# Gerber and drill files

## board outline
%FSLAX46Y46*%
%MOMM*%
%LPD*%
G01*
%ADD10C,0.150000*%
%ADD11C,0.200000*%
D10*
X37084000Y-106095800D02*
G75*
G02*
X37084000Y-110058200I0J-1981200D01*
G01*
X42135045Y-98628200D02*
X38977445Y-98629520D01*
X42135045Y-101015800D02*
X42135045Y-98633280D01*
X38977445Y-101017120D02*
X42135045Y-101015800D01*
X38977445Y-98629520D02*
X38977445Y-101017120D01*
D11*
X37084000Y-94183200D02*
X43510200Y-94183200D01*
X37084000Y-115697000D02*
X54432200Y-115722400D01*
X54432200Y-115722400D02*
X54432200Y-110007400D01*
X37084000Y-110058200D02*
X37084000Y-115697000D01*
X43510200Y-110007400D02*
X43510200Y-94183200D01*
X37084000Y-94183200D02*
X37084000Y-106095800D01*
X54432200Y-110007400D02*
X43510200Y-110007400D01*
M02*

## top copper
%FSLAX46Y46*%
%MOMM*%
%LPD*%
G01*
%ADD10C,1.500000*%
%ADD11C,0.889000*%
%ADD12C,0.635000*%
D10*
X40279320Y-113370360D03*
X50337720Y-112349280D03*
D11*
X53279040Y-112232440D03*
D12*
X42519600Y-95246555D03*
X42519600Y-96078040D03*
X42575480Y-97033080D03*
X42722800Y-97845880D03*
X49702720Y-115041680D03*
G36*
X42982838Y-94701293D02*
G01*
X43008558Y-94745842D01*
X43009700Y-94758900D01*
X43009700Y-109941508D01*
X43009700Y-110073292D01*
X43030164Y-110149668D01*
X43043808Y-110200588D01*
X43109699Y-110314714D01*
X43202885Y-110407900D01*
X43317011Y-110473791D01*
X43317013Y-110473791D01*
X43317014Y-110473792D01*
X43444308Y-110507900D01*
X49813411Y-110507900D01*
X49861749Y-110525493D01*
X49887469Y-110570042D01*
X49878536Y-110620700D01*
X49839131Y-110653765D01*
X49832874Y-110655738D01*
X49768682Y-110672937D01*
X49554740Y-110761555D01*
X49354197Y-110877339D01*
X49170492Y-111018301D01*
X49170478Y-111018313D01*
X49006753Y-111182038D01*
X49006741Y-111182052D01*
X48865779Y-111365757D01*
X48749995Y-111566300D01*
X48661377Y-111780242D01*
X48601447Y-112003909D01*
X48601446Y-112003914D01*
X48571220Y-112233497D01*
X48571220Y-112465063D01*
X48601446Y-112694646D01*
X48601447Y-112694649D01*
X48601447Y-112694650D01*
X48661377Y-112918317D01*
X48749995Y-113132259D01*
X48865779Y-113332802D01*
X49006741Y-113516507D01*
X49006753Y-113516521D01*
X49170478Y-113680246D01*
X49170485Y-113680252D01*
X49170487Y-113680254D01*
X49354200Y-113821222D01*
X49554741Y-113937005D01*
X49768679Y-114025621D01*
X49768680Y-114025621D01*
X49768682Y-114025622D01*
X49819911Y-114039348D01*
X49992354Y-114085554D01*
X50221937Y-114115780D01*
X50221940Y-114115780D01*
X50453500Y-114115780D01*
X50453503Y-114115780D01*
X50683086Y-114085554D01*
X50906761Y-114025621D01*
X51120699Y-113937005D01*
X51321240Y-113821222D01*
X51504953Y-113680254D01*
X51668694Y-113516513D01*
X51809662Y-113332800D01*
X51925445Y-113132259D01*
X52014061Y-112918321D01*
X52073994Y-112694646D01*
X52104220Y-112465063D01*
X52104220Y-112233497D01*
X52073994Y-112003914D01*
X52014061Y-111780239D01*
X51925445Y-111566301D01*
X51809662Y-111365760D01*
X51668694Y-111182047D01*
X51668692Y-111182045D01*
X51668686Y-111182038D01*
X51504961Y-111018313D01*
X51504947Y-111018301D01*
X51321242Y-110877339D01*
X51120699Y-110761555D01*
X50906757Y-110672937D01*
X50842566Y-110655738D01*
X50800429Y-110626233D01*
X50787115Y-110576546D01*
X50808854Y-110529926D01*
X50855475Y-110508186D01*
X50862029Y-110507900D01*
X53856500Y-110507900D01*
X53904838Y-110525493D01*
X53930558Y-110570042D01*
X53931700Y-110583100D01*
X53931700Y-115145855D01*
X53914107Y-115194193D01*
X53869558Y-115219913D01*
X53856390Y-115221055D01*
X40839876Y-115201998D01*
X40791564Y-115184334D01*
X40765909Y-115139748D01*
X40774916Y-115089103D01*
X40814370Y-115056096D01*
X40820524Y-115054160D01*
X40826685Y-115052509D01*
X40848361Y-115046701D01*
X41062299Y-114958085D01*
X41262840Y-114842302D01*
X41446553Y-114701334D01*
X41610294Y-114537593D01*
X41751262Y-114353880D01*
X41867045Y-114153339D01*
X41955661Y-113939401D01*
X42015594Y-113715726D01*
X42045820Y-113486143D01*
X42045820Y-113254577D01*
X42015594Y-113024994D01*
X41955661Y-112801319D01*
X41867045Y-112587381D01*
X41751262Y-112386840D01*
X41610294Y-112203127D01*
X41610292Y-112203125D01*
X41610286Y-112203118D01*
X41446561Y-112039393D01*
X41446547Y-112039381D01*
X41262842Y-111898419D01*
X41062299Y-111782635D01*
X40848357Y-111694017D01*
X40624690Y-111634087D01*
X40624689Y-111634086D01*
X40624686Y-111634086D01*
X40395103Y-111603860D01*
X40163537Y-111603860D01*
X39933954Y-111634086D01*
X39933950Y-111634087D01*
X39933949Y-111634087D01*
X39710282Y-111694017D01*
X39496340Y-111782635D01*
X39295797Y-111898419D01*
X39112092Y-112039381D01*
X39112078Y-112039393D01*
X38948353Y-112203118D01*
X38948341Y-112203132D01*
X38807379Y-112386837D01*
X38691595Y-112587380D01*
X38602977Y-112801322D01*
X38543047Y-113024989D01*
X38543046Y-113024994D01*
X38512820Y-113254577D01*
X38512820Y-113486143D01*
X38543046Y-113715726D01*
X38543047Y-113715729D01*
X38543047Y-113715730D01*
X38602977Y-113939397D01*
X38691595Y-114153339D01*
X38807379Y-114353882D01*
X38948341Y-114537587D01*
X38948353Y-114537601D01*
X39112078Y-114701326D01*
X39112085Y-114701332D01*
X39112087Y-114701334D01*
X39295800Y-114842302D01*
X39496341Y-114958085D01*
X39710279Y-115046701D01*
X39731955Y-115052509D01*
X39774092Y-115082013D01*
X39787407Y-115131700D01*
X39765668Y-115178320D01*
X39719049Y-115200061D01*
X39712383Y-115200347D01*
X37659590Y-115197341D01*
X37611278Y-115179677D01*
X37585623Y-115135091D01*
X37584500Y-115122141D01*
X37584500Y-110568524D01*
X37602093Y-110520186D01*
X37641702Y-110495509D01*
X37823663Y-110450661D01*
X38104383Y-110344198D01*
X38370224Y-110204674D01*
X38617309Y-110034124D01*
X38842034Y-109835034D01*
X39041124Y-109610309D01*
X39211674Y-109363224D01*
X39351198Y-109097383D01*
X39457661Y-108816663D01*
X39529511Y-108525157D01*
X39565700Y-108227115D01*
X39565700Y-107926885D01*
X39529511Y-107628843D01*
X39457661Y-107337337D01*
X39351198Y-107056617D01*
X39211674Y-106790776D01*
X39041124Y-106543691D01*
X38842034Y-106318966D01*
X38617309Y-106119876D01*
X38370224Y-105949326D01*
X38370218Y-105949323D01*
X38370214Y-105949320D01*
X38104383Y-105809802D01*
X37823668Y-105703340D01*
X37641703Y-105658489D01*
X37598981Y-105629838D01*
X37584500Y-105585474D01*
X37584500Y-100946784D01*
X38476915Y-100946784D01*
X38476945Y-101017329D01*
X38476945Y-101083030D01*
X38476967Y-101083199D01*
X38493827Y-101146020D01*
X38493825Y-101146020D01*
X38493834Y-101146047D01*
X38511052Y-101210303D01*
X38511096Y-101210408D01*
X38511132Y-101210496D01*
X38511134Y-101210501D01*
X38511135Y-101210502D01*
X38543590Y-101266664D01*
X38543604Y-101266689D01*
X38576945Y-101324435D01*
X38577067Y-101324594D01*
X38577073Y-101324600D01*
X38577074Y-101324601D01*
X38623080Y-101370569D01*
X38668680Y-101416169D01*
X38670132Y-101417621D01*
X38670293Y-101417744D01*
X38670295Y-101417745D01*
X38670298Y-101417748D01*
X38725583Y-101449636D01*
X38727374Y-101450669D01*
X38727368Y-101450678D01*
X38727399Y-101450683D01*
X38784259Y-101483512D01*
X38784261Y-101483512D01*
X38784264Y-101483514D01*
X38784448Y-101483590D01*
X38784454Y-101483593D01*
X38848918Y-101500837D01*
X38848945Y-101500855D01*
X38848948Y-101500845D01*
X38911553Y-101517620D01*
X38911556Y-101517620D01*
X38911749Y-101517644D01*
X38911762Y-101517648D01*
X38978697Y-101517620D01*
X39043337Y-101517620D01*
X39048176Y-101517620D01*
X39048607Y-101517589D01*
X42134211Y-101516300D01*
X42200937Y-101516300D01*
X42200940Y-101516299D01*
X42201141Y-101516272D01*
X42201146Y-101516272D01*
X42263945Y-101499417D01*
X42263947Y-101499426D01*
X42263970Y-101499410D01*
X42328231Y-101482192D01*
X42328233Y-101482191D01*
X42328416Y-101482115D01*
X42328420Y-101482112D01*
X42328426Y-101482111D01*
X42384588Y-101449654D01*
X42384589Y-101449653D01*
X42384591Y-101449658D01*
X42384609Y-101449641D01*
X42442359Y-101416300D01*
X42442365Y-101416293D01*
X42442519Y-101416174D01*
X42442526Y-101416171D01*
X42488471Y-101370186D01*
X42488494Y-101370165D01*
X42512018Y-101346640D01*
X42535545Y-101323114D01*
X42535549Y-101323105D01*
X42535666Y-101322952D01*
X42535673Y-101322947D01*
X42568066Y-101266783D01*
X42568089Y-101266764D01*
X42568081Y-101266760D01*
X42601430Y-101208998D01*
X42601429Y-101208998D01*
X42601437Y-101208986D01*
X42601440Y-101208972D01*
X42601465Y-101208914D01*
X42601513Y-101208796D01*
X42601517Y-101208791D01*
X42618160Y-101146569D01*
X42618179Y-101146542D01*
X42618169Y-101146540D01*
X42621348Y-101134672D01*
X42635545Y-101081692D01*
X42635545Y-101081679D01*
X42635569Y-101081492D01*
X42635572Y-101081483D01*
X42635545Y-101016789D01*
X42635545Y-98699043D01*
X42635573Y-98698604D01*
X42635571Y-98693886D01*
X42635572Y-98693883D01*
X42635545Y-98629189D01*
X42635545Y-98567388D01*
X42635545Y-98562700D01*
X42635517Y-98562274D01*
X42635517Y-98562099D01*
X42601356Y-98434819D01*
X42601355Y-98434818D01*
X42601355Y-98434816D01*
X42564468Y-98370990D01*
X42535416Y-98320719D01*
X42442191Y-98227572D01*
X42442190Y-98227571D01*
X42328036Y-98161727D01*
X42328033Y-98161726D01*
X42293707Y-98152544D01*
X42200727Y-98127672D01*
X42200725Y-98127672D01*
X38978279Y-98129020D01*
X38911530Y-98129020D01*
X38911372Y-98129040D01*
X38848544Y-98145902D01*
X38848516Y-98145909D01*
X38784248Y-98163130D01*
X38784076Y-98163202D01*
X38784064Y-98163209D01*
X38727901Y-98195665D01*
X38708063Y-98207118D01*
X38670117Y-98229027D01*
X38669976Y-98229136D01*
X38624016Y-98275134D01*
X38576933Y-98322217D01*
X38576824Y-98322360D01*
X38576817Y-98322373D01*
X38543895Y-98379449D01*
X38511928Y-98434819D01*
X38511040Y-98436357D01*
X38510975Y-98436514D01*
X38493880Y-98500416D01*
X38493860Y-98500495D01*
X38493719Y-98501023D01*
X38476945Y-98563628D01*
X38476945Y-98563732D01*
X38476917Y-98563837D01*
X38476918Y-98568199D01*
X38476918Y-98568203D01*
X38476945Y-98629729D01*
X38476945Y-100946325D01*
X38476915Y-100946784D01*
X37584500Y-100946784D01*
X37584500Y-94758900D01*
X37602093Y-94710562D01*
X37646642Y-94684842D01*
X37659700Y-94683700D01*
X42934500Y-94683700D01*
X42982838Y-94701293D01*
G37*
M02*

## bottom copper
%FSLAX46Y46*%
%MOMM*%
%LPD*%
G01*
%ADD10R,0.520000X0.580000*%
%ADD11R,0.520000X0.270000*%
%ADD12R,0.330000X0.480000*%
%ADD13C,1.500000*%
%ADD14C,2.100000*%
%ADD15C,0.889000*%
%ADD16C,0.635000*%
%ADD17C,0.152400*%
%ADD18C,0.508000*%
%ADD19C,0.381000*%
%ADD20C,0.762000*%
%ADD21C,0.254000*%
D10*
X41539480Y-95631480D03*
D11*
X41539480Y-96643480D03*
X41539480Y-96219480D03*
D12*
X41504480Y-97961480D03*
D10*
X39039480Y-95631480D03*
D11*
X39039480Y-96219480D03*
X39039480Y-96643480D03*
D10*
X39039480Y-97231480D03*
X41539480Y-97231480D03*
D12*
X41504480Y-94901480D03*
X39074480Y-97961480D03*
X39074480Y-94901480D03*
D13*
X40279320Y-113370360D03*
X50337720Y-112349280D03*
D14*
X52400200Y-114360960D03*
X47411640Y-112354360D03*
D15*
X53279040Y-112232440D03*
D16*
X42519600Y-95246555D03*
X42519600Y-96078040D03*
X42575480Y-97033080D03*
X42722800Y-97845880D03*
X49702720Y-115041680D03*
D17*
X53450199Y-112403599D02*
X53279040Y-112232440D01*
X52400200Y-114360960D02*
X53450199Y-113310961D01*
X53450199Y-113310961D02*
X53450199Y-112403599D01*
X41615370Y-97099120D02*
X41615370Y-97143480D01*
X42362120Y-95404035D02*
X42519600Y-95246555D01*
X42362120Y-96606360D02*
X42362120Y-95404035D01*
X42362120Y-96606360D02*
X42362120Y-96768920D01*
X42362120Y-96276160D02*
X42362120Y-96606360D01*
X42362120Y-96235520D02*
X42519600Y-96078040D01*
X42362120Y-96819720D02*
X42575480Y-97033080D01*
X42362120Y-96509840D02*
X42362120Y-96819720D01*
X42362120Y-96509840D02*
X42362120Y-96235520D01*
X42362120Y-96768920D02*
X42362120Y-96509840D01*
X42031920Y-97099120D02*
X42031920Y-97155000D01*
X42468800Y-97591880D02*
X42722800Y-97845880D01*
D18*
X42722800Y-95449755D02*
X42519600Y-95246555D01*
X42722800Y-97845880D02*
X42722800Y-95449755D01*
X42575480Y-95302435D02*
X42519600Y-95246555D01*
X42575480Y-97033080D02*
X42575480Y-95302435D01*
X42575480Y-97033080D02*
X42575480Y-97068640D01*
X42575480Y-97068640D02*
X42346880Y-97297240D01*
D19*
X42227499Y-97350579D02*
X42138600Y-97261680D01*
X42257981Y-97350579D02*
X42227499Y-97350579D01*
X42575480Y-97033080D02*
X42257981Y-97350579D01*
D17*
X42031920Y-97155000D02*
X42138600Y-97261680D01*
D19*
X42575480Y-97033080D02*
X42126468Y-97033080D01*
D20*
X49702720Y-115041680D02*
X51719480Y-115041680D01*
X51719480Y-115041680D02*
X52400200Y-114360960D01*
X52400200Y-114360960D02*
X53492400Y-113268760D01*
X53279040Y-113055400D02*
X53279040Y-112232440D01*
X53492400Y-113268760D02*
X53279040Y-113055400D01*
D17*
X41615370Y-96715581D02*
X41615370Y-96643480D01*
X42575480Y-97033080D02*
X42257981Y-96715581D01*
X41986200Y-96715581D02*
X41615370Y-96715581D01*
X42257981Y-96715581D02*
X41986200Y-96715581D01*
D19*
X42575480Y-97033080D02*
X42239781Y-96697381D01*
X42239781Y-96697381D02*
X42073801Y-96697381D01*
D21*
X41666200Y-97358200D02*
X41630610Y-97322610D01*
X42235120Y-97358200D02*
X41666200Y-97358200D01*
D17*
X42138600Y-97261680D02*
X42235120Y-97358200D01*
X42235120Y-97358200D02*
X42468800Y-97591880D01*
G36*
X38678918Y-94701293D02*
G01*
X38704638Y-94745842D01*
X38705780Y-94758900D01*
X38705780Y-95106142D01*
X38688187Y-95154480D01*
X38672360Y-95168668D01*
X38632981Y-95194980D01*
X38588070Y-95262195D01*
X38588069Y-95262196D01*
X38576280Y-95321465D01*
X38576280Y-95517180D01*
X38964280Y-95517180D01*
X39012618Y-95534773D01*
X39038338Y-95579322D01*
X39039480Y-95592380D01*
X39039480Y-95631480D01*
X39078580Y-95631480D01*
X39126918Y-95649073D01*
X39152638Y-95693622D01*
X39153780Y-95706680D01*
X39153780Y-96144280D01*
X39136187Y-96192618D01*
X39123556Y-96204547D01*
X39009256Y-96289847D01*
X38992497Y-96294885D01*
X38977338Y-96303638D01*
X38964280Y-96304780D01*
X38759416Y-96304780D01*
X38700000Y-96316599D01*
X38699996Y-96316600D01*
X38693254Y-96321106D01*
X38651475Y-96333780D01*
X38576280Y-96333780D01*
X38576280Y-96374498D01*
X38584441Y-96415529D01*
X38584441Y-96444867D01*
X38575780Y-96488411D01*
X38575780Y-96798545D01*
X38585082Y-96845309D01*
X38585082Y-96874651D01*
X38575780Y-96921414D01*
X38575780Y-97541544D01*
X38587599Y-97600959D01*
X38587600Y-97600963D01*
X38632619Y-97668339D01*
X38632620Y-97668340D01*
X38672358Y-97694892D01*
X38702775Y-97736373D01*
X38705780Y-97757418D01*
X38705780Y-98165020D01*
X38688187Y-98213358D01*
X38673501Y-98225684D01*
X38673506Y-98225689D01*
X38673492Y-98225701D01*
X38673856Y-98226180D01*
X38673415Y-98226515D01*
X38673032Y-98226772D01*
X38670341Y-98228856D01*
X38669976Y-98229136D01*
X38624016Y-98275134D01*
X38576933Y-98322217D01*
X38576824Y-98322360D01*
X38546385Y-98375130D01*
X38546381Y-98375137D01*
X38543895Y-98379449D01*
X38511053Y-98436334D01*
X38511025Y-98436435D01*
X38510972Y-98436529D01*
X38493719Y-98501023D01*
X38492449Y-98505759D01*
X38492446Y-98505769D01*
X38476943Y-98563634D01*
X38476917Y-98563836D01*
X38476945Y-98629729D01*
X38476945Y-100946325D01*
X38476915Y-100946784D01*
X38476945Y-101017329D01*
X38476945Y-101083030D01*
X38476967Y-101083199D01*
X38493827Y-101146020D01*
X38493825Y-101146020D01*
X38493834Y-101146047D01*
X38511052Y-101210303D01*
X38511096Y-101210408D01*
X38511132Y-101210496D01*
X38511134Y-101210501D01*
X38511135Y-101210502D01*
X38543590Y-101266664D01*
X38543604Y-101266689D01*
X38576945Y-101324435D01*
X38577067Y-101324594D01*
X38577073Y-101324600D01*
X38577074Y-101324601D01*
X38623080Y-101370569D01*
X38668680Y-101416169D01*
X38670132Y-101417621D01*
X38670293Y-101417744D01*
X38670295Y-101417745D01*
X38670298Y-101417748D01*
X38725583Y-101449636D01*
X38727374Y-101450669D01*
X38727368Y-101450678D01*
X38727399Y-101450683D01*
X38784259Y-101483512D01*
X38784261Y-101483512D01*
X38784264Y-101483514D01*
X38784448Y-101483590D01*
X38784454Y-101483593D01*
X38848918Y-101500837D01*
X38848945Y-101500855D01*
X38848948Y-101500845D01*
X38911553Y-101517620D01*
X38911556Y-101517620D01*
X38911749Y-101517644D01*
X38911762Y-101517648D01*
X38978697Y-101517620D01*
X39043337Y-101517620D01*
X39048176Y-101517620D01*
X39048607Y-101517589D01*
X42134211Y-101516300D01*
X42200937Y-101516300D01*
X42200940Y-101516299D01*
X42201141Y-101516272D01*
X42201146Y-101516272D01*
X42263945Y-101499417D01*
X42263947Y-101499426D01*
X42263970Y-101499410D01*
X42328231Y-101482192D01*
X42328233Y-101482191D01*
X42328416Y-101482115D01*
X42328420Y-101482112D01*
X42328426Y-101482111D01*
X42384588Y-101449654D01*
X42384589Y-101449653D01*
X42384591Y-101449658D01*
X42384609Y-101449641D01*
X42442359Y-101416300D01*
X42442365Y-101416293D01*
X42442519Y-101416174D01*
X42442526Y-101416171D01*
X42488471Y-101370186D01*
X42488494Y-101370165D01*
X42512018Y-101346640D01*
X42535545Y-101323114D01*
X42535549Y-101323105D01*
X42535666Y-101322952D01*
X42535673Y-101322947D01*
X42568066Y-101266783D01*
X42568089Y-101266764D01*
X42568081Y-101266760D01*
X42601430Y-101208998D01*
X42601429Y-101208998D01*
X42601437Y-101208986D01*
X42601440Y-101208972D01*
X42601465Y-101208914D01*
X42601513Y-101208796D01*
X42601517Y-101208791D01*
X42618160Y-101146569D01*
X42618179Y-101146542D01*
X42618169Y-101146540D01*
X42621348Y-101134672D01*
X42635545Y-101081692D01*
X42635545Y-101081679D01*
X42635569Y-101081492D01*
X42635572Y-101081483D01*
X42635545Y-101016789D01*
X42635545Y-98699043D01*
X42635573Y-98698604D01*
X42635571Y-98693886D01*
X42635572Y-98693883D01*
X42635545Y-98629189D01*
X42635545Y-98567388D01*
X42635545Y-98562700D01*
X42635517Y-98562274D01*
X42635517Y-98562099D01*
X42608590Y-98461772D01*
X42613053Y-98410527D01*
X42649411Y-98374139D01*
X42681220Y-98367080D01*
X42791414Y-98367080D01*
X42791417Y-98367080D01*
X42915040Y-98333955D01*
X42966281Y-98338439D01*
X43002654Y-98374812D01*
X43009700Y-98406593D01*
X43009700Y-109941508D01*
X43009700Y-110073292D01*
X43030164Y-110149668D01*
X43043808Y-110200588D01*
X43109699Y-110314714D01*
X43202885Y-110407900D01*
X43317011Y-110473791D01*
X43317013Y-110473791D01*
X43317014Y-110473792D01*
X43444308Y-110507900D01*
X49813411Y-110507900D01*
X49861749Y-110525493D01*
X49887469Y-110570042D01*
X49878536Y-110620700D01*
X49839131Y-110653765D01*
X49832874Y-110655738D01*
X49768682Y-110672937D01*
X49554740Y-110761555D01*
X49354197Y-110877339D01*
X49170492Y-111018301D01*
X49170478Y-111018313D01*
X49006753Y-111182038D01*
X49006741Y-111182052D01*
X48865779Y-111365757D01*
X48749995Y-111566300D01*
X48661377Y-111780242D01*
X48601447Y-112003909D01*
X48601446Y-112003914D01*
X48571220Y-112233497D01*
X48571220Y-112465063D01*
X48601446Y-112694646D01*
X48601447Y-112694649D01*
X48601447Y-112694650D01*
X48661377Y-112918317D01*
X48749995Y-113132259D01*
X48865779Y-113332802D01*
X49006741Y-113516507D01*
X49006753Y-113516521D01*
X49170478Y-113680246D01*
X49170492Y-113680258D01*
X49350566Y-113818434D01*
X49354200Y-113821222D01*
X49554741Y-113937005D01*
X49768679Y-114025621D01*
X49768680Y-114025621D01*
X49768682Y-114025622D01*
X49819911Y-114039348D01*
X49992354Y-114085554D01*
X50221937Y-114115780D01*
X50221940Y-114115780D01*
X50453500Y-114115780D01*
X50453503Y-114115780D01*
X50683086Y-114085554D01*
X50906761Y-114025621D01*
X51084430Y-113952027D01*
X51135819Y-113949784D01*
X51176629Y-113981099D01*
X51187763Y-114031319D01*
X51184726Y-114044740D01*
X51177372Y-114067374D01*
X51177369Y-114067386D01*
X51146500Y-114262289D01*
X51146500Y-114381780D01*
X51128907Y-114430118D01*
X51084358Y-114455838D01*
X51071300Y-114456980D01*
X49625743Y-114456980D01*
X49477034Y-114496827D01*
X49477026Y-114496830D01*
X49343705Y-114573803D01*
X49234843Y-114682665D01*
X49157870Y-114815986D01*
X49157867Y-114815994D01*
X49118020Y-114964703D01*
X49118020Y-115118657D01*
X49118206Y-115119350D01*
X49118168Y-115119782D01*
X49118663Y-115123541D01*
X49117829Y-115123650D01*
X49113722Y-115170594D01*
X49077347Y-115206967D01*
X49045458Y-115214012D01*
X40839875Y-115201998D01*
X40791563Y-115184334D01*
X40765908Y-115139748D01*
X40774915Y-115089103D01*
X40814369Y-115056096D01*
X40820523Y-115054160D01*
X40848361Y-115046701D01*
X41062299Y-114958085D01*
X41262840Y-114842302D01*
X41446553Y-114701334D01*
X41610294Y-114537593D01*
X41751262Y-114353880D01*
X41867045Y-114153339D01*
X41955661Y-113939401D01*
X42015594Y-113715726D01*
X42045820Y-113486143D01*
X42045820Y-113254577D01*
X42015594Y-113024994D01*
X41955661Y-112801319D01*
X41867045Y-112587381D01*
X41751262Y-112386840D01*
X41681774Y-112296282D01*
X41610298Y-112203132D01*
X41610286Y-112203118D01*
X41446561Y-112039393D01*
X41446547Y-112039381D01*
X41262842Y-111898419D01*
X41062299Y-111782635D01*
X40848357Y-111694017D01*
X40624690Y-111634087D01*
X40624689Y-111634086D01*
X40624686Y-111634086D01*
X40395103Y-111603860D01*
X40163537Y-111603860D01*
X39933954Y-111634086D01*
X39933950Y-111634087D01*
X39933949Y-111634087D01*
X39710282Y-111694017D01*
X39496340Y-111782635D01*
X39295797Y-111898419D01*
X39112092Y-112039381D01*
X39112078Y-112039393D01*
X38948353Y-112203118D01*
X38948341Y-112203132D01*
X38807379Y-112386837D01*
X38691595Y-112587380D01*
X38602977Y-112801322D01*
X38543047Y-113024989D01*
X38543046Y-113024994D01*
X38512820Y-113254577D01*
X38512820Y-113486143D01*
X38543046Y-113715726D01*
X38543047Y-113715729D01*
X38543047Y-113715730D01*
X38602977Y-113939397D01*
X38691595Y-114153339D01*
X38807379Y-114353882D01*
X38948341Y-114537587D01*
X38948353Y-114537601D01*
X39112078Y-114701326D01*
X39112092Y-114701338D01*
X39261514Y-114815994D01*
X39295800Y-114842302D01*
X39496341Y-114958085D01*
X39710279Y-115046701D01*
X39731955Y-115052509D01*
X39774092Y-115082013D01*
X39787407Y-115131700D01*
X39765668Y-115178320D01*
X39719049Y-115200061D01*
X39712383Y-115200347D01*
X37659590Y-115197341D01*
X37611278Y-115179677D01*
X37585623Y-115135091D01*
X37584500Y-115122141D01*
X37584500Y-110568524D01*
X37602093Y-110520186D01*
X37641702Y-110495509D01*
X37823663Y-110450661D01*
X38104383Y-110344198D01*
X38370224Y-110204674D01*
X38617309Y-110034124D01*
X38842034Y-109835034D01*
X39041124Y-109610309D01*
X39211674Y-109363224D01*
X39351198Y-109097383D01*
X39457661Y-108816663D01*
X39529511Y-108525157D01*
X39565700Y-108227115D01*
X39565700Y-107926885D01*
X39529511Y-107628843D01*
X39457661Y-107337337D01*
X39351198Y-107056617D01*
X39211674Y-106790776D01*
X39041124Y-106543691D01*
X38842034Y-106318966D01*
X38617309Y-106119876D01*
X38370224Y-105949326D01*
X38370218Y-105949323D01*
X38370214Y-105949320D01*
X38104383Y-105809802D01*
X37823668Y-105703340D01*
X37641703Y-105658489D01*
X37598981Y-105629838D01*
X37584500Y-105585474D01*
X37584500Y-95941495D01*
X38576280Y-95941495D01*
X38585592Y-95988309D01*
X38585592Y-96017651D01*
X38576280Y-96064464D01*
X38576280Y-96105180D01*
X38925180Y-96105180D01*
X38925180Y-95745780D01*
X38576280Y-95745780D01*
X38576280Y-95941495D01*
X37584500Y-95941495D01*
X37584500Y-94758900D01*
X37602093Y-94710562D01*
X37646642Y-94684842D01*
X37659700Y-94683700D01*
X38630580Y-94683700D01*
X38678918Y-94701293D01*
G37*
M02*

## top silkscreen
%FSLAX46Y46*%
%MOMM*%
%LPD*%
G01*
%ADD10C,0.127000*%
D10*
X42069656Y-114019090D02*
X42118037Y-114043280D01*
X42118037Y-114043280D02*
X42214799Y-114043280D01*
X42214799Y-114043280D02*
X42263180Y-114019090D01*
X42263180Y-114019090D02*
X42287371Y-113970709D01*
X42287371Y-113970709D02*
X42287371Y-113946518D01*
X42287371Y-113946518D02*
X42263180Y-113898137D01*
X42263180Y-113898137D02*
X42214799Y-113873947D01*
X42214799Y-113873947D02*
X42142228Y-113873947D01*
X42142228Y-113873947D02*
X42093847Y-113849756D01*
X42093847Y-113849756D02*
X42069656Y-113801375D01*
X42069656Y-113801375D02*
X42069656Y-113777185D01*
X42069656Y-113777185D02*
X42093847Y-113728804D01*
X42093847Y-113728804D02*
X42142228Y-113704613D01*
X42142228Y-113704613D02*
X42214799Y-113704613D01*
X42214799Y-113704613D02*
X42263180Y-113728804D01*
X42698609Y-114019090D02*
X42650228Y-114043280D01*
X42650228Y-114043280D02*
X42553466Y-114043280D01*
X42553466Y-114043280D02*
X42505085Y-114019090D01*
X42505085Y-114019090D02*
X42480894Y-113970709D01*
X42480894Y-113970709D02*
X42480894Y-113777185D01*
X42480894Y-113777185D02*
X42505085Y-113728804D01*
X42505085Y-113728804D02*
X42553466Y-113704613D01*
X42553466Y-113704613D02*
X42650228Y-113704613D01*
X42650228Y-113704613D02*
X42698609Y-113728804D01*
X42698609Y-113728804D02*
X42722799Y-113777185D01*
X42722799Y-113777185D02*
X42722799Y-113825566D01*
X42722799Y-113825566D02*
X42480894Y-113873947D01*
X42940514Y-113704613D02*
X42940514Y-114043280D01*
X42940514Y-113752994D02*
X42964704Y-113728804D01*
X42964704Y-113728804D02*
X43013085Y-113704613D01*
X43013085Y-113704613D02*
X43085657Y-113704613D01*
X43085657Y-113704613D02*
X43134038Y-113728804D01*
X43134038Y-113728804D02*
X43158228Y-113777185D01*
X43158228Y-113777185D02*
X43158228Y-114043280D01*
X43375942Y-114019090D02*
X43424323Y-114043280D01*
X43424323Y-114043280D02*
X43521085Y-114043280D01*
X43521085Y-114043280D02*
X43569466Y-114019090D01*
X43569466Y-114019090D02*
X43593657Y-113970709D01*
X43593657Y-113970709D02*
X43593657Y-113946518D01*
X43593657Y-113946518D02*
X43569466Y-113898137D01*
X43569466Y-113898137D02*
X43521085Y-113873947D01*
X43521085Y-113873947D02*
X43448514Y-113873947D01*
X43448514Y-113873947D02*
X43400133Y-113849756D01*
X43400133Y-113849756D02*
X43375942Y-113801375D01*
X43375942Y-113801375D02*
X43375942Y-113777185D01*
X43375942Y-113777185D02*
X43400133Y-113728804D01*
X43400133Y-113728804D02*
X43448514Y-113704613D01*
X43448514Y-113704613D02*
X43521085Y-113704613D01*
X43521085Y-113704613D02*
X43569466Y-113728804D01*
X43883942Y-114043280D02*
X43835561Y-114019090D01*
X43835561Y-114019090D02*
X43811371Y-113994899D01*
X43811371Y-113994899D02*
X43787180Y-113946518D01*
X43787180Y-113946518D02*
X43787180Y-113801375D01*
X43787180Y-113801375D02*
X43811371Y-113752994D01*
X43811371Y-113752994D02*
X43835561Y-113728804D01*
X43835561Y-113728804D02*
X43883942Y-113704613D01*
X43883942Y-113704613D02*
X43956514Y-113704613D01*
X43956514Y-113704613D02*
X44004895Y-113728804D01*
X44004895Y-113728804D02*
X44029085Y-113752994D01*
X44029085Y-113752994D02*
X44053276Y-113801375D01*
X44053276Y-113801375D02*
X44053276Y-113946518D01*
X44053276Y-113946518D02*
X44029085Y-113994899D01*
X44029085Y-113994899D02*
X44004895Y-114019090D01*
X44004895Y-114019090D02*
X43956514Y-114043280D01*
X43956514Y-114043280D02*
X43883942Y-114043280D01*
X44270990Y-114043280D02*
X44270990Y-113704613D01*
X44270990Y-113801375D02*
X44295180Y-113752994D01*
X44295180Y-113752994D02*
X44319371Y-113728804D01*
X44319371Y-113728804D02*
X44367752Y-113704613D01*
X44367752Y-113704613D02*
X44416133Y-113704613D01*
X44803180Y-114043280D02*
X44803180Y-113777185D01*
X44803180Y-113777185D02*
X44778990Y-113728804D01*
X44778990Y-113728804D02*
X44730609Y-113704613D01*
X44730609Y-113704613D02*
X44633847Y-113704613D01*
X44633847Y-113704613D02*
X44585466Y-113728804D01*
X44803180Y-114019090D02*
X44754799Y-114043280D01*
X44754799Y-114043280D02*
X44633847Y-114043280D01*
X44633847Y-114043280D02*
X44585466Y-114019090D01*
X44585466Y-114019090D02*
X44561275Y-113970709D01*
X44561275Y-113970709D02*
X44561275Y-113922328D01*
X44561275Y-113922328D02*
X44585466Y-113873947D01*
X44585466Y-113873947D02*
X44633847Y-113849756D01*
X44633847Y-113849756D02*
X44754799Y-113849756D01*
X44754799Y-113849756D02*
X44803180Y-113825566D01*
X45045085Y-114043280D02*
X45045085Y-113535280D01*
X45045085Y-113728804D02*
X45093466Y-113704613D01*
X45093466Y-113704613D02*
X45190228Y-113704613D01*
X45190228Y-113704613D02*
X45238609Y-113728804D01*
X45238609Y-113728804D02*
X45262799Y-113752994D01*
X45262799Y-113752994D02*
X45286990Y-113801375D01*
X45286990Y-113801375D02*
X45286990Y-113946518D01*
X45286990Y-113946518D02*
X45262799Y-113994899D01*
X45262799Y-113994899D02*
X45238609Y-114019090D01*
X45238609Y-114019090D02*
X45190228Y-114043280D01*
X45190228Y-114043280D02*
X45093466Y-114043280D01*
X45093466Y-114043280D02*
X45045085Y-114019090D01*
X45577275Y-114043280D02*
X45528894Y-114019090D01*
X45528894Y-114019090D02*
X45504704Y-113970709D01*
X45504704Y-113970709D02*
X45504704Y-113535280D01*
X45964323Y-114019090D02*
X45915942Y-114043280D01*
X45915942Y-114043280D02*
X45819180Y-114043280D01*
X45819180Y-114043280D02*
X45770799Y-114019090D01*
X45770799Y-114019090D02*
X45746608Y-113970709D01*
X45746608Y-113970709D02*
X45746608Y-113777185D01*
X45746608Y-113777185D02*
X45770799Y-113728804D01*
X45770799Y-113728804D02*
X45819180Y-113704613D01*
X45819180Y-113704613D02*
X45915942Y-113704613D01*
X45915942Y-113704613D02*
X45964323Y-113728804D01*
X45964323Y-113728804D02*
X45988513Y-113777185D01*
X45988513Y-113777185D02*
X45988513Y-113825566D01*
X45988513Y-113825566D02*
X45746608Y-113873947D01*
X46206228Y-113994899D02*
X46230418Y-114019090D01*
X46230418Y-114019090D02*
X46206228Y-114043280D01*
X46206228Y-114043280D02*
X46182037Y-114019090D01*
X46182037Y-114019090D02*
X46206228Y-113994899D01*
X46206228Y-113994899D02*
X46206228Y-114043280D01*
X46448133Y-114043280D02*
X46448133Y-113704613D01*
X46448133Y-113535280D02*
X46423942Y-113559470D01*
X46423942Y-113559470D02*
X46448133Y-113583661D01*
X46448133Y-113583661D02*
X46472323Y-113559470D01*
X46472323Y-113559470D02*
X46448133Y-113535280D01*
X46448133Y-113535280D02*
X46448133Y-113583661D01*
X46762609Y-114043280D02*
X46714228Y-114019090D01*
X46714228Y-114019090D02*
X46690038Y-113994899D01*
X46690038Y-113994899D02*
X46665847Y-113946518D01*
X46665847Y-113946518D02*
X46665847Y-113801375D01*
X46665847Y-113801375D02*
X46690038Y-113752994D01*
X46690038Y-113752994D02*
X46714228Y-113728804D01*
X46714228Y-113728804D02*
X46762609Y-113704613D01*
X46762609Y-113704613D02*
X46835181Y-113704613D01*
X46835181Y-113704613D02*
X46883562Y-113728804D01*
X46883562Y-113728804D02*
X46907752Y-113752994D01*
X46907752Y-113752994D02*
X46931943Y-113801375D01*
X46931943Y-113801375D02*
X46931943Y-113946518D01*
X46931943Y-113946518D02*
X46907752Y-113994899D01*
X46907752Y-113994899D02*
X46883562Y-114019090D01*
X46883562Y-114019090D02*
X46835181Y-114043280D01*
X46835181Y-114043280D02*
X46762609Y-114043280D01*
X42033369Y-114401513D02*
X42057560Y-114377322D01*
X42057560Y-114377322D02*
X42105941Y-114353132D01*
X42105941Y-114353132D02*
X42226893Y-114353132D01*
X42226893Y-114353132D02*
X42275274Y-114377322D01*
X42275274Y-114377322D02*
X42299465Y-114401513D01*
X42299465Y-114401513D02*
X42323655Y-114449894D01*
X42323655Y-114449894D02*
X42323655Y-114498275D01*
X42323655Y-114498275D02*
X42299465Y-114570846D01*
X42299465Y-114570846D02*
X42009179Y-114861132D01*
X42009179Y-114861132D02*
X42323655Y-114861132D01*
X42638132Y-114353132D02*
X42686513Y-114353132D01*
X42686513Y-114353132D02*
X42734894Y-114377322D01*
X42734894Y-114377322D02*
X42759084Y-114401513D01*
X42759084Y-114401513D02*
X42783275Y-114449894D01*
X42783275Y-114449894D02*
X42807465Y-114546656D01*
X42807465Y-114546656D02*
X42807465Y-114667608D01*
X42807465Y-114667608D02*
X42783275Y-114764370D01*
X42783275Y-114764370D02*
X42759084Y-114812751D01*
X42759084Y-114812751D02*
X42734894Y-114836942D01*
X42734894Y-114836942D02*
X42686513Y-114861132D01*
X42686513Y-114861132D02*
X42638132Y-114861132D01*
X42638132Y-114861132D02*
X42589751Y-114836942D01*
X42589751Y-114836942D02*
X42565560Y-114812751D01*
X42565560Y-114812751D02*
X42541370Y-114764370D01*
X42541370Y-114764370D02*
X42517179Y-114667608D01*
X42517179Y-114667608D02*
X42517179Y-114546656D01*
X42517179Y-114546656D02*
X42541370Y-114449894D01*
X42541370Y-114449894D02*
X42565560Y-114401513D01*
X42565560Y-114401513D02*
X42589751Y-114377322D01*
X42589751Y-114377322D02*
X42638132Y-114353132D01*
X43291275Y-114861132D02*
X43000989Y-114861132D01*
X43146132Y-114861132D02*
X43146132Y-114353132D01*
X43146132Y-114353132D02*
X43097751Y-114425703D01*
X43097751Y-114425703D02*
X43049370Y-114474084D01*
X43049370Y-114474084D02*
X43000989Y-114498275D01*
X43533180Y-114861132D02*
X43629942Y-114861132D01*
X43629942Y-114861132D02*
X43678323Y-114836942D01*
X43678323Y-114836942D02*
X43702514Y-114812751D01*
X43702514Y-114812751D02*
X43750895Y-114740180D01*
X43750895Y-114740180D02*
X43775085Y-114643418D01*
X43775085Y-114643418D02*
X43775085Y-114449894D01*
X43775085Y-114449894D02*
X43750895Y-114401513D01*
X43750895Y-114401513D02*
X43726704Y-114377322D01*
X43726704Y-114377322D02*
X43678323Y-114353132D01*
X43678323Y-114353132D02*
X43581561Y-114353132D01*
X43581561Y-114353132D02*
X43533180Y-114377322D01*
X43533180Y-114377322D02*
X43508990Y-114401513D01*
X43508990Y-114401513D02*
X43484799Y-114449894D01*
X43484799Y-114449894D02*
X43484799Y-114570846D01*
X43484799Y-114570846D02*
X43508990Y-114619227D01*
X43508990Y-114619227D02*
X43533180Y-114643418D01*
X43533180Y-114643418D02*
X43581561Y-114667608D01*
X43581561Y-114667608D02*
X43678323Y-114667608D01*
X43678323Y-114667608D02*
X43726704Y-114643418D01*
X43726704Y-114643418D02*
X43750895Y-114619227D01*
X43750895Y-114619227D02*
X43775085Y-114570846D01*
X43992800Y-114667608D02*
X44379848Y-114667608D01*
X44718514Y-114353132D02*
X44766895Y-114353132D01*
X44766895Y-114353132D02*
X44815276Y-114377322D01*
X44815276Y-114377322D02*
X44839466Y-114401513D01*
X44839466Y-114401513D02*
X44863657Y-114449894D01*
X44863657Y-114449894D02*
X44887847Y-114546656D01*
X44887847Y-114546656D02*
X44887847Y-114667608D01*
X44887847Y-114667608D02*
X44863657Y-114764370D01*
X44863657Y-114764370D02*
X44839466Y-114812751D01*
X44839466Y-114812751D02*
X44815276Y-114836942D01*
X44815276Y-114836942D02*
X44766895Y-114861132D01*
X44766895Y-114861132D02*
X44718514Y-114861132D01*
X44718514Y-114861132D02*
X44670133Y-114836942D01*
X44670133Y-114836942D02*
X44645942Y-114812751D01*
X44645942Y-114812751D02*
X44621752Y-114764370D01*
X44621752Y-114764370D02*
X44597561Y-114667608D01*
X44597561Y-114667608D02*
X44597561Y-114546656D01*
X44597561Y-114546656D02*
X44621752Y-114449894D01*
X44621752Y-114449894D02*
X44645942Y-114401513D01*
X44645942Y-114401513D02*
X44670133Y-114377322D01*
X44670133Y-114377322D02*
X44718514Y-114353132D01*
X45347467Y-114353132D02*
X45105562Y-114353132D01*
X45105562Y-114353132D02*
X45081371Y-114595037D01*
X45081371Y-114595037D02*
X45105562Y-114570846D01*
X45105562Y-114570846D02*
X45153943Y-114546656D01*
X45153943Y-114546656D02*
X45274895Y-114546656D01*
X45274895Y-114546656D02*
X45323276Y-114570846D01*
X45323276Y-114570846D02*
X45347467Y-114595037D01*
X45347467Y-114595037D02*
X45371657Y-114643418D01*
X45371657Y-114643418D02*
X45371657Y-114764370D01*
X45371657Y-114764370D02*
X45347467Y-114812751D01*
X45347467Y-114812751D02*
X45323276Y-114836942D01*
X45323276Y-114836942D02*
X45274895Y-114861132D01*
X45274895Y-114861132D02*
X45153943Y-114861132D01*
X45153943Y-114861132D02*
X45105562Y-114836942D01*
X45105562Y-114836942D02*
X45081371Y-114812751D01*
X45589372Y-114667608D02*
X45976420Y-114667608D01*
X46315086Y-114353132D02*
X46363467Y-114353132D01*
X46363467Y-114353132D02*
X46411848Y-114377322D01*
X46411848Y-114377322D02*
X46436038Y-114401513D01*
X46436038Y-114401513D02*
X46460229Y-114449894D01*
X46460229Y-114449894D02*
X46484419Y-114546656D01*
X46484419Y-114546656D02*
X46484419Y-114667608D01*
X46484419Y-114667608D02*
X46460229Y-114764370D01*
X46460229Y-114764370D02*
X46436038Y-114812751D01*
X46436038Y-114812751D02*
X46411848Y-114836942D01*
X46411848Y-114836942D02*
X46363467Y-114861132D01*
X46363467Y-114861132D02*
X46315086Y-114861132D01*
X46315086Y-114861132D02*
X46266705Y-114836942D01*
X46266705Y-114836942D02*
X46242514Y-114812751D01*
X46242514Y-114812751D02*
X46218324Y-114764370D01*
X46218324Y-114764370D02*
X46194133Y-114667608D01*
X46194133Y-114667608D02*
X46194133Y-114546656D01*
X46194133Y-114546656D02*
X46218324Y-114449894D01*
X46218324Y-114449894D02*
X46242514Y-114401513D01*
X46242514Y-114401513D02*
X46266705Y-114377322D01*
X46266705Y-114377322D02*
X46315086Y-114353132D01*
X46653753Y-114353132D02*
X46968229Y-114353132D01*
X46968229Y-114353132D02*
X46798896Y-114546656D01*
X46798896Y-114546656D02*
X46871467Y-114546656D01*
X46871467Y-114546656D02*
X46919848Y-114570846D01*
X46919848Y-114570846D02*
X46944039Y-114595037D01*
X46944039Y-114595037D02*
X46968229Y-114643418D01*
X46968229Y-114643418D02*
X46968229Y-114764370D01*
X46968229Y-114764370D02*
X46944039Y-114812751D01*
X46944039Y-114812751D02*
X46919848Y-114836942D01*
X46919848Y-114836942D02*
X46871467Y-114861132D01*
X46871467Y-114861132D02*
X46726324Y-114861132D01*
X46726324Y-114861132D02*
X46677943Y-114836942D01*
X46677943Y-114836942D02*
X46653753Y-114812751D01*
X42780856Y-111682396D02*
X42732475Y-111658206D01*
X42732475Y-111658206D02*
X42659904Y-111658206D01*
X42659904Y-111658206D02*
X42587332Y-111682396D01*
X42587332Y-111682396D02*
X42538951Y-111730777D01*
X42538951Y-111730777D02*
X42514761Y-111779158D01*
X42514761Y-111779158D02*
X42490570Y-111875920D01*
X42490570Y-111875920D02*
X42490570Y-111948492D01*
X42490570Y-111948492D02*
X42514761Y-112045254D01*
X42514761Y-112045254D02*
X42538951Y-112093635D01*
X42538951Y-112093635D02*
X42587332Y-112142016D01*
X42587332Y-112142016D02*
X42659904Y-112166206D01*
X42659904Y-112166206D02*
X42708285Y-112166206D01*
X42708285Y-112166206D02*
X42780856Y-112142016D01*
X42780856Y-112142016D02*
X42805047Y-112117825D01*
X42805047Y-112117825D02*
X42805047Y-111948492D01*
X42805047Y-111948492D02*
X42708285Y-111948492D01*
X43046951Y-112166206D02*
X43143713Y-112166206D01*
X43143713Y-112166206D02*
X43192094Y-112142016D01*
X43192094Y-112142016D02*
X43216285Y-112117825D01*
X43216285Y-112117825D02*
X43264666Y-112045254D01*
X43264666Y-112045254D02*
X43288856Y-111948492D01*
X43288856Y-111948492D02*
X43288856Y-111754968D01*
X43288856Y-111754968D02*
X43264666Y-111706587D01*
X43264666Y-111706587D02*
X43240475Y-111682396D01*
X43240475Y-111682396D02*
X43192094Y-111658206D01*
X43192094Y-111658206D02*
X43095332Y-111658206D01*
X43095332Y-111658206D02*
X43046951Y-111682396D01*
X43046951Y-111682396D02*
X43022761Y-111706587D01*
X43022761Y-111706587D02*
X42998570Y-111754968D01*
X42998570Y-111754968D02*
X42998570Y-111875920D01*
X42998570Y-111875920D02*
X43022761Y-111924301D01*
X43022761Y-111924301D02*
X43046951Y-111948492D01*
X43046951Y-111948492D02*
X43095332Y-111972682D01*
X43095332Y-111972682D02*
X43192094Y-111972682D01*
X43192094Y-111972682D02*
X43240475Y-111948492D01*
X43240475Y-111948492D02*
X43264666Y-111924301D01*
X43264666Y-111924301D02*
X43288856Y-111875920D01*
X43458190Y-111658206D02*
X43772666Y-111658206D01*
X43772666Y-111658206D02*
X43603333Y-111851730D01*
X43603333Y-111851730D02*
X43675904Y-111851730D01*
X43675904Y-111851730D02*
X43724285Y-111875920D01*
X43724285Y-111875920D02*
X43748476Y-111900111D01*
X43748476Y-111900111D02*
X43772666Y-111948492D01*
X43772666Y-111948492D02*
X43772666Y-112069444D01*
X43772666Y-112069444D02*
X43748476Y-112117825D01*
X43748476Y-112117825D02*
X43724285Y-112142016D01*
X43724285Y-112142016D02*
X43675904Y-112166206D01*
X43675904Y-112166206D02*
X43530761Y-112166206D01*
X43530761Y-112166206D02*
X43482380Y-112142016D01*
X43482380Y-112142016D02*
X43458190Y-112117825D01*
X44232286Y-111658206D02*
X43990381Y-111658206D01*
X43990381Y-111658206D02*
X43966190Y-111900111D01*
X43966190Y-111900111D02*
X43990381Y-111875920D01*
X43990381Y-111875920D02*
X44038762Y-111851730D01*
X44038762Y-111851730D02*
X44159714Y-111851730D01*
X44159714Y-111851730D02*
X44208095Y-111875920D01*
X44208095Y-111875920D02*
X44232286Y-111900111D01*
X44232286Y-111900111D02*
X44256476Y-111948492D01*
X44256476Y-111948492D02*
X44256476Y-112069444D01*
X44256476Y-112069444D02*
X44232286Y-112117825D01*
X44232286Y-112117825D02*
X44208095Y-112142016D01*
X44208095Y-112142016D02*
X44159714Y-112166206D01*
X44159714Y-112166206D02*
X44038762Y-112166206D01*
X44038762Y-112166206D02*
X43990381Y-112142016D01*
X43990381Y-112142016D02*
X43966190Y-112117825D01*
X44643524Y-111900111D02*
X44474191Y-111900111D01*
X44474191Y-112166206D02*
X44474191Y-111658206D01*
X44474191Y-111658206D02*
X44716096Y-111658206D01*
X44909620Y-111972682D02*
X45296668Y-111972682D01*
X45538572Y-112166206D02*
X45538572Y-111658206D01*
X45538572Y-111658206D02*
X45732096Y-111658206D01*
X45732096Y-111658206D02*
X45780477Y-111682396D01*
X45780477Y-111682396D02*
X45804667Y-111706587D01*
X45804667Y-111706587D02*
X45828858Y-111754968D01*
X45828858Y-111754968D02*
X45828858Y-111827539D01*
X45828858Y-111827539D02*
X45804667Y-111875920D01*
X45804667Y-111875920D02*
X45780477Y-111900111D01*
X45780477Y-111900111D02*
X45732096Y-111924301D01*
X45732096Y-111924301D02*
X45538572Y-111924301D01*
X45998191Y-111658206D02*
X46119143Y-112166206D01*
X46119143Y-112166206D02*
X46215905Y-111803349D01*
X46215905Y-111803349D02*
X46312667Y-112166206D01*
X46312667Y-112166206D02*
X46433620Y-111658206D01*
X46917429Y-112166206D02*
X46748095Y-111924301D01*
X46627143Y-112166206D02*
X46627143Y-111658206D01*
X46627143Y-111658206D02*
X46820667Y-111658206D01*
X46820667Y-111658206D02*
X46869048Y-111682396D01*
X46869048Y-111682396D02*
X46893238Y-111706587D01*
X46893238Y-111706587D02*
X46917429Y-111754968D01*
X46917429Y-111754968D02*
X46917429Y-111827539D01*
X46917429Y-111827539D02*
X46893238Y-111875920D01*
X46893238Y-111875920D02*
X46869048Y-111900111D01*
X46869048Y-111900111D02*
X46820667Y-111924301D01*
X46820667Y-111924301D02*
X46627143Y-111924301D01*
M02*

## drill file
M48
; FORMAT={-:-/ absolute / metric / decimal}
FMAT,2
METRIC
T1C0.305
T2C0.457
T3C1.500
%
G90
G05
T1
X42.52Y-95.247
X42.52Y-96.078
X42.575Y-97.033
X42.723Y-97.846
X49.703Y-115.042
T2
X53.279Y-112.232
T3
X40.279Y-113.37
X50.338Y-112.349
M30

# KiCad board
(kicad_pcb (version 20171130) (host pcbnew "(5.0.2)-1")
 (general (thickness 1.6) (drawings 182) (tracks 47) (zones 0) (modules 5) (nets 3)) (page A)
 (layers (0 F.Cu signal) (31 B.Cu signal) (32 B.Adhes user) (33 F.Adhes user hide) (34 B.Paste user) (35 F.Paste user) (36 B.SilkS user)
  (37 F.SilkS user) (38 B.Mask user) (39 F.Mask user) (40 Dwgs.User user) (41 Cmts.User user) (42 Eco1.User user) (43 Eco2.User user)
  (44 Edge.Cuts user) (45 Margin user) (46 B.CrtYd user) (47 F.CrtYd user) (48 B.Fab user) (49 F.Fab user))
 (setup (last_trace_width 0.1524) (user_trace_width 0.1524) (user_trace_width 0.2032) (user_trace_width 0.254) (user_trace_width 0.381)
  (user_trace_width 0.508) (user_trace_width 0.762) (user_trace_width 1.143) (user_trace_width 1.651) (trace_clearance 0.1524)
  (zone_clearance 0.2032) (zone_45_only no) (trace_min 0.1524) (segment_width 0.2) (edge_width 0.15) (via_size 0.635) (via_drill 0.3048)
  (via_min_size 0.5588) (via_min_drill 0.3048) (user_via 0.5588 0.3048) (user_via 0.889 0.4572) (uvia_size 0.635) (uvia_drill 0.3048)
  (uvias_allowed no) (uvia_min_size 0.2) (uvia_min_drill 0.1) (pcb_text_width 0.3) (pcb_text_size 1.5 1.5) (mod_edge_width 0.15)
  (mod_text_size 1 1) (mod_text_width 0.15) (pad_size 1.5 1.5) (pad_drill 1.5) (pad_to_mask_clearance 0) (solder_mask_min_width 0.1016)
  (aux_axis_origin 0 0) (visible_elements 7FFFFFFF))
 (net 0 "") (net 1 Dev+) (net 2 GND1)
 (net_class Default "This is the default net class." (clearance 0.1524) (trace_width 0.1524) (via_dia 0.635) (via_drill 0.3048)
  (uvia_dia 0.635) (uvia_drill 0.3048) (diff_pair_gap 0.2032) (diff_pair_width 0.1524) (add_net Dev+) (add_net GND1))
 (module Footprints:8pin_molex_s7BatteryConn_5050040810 (layer B.Cu) (at 40.28948 96.43148)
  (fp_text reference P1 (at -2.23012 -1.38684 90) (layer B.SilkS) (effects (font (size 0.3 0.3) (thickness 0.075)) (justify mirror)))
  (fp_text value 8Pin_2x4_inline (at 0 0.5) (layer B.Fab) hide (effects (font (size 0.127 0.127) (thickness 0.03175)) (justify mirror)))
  (pad 5 smd rect (at 1.25 -0.8) (size 0.52 0.58) (layers B.Cu B.Paste B.Mask))
  (pad 7 smd rect (at 1.25 0.212) (size 0.52 0.27) (layers B.Cu B.Paste B.Mask) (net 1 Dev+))
  (pad 6 smd rect (at 1.25 -0.212) (size 0.52 0.27) (layers B.Cu B.Paste B.Mask))
  (pad "" smd rect (at 1.215 1.53) (size 0.33 0.48) (layers B.Cu B.Paste B.Mask))
  (pad 4 smd rect (at -1.25 -0.8) (size 0.52 0.58) (layers B.Cu B.Paste B.Mask) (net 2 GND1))
  (pad 3 smd rect (at -1.25 -0.212) (size 0.52 0.27) (layers B.Cu B.Paste B.Mask) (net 2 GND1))
  (pad 2 smd rect (at -1.25 0.212) (size 0.52 0.27) (layers B.Cu B.Paste B.Mask))
  (pad 1 smd rect (at -1.25 0.8) (size 0.52 0.58) (layers B.Cu B.Paste B.Mask))
  (pad 8 smd rect (at 1.25 0.8) (size 0.52 0.58) (layers B.Cu B.Paste B.Mask) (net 1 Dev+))
  (pad "" smd rect (at 1.215 -1.53) (size 0.33 0.48) (layers B.Cu B.Paste B.Mask))
  (pad "" smd rect (at -1.215 1.53) (size 0.33 0.48) (layers B.Cu B.Paste B.Mask))
  (pad "" smd rect (at -1.215 -1.53) (size 0.33 0.48) (layers B.Cu B.Paste B.Mask)))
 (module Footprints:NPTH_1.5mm (layer F.Cu) (at 40.27932 113.37036)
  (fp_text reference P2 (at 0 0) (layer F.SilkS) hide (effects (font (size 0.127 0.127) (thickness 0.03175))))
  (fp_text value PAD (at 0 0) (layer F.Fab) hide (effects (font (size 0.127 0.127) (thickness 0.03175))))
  (pad "" thru_hole circle (at 0 0) (size 1.5 1.5) (drill 1.5) (layers *.Cu *.Mask) (clearance 1.016)))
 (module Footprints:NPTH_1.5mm (layer F.Cu) (at 50.33772 112.34928)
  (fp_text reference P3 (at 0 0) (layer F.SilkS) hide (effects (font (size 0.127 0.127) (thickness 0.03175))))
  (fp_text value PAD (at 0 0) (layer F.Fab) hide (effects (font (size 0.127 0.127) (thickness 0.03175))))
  (pad "" thru_hole circle (at 0 0) (size 1.5 1.5) (drill 1.5) (layers *.Cu *.Mask) (clearance 1.016)))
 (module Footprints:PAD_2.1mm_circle (layer B.Cu) (at 52.4002 114.36096)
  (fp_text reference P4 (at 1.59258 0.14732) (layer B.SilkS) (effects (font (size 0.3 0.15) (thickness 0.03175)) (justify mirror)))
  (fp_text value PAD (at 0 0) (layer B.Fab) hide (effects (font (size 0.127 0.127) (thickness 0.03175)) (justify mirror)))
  (pad 1 smd circle (at 0 0) (size 2.1 2.1) (layers B.Cu B.Paste B.Mask) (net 1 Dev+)))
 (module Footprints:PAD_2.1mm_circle (layer B.Cu) (at 47.41164 112.35436)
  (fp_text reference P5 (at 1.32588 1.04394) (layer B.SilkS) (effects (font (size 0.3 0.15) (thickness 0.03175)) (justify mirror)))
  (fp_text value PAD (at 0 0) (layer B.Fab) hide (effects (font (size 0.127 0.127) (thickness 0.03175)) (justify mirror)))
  (pad 1 smd circle (at 0 0) (size 2.1 2.1) (layers B.Cu B.Paste B.Mask) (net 2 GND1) (zone_connect 2)))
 (gr_arc (start 37.084 108.077) (end 37.084 110.0582) (angle -180) (layer Edge.Cuts) (width 0.15))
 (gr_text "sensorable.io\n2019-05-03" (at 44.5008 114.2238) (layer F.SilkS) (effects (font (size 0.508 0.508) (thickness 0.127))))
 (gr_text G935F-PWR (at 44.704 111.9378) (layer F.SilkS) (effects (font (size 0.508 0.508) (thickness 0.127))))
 (gr_line (start 42.135045 98.6282) (end 38.977445 98.62952) (layer Edge.Cuts) (width 0.15))
 (gr_line (start 42.135045 101.0158) (end 42.135045 98.63328) (layer Edge.Cuts) (width 0.15))
 (gr_line (start 38.977445 101.01712) (end 42.135045 101.0158) (layer Edge.Cuts) (width 0.15))
 (gr_line (start 38.977445 98.62952) (end 38.977445 101.01712) (layer Edge.Cuts) (width 0.15))
 (gr_line (start 37.084 94.1832) (end 43.5102 94.1832) (layer Edge.Cuts) (width 0.2))
 (gr_line (start 37.084 115.697) (end 54.4322 115.7224) (layer Edge.Cuts) (width 0.2))
 (gr_line (start 54.4322 115.7224) (end 54.4322 110.0074) (layer Edge.Cuts) (width 0.2))
 (gr_line (start 37.084 110.0582) (end 37.084 115.697) (layer Edge.Cuts) (width 0.2))
 (gr_line (start 43.5102 110.0074) (end 43.5102 94.1832) (layer Edge.Cuts) (width 0.2))
 (gr_line (start 37.084 94.1832) (end 37.084 106.0958) (layer Edge.Cuts) (width 0.2))
 (gr_line (start 54.4322 110.0074) (end 43.5102 110.0074) (layer Edge.Cuts) (width 0.2))
 (via (at 53.27904 112.23244) (size 0.889) (drill 0.4572) (layers F.Cu B.Cu) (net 1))
 (segment (start 53.450199 112.403599) (end 53.27904 112.23244) (width 0.1524) (layer B.Cu) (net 1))
 (segment (start 52.4002 114.36096) (end 53.450199 113.310961) (width 0.1524) (layer B.Cu) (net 1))
 (segment (start 53.450199 113.310961) (end 53.450199 112.403599) (width 0.1524) (layer B.Cu) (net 1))
 (segment (start 41.61537 97.09912) (end 41.61537 97.14348) (width 0.1524) (layer B.Cu) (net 1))
 (via (at 42.5196 95.246555) (size 0.635) (drill 0.3048) (layers F.Cu B.Cu) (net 1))
 (segment (start 42.36212 95.404035) (end 42.5196 95.246555) (width 0.1524) (layer B.Cu) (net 1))
 (segment (start 42.36212 96.60636) (end 42.36212 95.404035) (width 0.1524) (layer B.Cu) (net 1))
 (segment (start 42.36212 96.60636) (end 42.36212 96.76892) (width 0.1524) (layer B.Cu) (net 1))
 (segment (start 42.36212 96.27616) (end 42.36212 96.60636) (width 0.1524) (layer B.Cu) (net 1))
 (via (at 42.5196 96.07804) (size 0.635) (drill 0.3048) (layers F.Cu B.Cu) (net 1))
 (segment (start 42.36212 96.23552) (end 42.5196 96.07804) (width 0.1524) (layer B.Cu) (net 1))
 (via (at 42.57548 97.03308) (size 0.635) (drill 0.3048) (layers F.Cu B.Cu) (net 1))
 (segment (start 42.36212 96.81972) (end 42.57548 97.03308) (width 0.1524) (layer B.Cu) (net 1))
 (segment (start 42.36212 96.50984) (end 42.36212 96.81972) (width 0.1524) (layer B.Cu) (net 1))
 (segment (start 42.36212 96.50984) (end 42.36212 96.23552) (width 0.1524) (layer B.Cu) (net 1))
 (segment (start 42.36212 96.76892) (end 42.36212 96.50984) (width 0.1524) (layer B.Cu) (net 1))
 (segment (start 42.03192 97.09912) (end 42.03192 97.155) (width 0.1524) (layer B.Cu) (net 1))
 (segment (start 42.4688 97.59188) (end 42.7228 97.84588) (width 0.1524) (layer B.Cu) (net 1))
 (via (at 42.7228 97.84588) (size 0.635) (drill 0.3048) (layers F.Cu B.Cu) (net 1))
 (segment (start 42.7228 95.449755) (end 42.5196 95.246555) (width 0.508) (layer B.Cu) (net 1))
 (segment (start 42.7228 97.84588) (end 42.7228 95.449755) (width 0.508) (layer B.Cu) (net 1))
 (segment (start 42.57548 95.302435) (end 42.5196 95.246555) (width 0.508) (layer B.Cu) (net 1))
 (segment (start 42.57548 97.03308) (end 42.57548 95.302435) (width 0.508) (layer B.Cu) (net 1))
 (segment (start 42.57548 97.03308) (end 42.57548 97.06864) (width 0.508) (layer B.Cu) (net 1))
 (segment (start 42.57548 97.06864) (end 42.34688 97.29724) (width 0.508) (layer B.Cu) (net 1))
 (segment (start 42.227499 97.350579) (end 42.1386 97.26168) (width 0.381) (layer B.Cu) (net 1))
 (segment (start 42.257981 97.350579) (end 42.227499 97.350579) (width 0.381) (layer B.Cu) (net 1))
 (segment (start 42.57548 97.03308) (end 42.257981 97.350579) (width 0.381) (layer B.Cu) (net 1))
 (segment (start 42.03192 97.155) (end 42.1386 97.26168) (width 0.1524) (layer B.Cu) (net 1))
 (segment (start 42.57548 97.03308) (end 42.126468 97.03308) (width 0.381) (layer B.Cu) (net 1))
 (via (at 49.70272 115.04168) (size 0.635) (drill 0.3048) (layers F.Cu B.Cu) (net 1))
 (segment (start 49.70272 115.04168) (end 51.71948 115.04168) (width 0.762) (layer B.Cu) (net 1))
 (segment (start 51.71948 115.04168) (end 52.4002 114.36096) (width 0.762) (layer B.Cu) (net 1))
 (segment (start 52.4002 114.36096) (end 53.4924 113.26876) (width 0.762) (layer B.Cu) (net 1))
 (segment (start 53.27904 113.0554) (end 53.27904 112.23244) (width 0.762) (layer B.Cu) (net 1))
 (segment (start 53.4924 113.26876) (end 53.27904 113.0554) (width 0.762) (layer B.Cu) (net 1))
 (segment (start 41.61537 96.715581) (end 41.61537 96.64348) (width 0.1524) (layer B.Cu) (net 1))
 (segment (start 42.57548 97.03308) (end 42.257981 96.715581) (width 0.1524) (layer B.Cu) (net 1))
 (segment (start 41.9862 96.715581) (end 41.61537 96.715581) (width 0.1524) (layer B.Cu) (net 1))
 (segment (start 42.257981 96.715581) (end 41.9862 96.715581) (width 0.1524) (layer B.Cu) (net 1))
 (segment (start 42.57548 97.03308) (end 42.239781 96.697381) (width 0.381) (layer B.Cu) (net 1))
 (segment (start 42.239781 96.697381) (end 42.073801 96.697381) (width 0.381) (layer B.Cu) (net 1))
 (segment (start 41.6662 97.3582) (end 41.63061 97.32261) (width 0.254) (layer B.Cu) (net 1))
 (segment (start 42.23512 97.3582) (end 41.6662 97.3582) (width 0.254) (layer B.Cu) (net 1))
 (segment (start 42.1386 97.26168) (end 42.23512 97.3582) (width 0.1524) (layer B.Cu) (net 1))
 (segment (start 42.23512 97.3582) (end 42.4688 97.59188) (width 0.1524) (layer B.Cu) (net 1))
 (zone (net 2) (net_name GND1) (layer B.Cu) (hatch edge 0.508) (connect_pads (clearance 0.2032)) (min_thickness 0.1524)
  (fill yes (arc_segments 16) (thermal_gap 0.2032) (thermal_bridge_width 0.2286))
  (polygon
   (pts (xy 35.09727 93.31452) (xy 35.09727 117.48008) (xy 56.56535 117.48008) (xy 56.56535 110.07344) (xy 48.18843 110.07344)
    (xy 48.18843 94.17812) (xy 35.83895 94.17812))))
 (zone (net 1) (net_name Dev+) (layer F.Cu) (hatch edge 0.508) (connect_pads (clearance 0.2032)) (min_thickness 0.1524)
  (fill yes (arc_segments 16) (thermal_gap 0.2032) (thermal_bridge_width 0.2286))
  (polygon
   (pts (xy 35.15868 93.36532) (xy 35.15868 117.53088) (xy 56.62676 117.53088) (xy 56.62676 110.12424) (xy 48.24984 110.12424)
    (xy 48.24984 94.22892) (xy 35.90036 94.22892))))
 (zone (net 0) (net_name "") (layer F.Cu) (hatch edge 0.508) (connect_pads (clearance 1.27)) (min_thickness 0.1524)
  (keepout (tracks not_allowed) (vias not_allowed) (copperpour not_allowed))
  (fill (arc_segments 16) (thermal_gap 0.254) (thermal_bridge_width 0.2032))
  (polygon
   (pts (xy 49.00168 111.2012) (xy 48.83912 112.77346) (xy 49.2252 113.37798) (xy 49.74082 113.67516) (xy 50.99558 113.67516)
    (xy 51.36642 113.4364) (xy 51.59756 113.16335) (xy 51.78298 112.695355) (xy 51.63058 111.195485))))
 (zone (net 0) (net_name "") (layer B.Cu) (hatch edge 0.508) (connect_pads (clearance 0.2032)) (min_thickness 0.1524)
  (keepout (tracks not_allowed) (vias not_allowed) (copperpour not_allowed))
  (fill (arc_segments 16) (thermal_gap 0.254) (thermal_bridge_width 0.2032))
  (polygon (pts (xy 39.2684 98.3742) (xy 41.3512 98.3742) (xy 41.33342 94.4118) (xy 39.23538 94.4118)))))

